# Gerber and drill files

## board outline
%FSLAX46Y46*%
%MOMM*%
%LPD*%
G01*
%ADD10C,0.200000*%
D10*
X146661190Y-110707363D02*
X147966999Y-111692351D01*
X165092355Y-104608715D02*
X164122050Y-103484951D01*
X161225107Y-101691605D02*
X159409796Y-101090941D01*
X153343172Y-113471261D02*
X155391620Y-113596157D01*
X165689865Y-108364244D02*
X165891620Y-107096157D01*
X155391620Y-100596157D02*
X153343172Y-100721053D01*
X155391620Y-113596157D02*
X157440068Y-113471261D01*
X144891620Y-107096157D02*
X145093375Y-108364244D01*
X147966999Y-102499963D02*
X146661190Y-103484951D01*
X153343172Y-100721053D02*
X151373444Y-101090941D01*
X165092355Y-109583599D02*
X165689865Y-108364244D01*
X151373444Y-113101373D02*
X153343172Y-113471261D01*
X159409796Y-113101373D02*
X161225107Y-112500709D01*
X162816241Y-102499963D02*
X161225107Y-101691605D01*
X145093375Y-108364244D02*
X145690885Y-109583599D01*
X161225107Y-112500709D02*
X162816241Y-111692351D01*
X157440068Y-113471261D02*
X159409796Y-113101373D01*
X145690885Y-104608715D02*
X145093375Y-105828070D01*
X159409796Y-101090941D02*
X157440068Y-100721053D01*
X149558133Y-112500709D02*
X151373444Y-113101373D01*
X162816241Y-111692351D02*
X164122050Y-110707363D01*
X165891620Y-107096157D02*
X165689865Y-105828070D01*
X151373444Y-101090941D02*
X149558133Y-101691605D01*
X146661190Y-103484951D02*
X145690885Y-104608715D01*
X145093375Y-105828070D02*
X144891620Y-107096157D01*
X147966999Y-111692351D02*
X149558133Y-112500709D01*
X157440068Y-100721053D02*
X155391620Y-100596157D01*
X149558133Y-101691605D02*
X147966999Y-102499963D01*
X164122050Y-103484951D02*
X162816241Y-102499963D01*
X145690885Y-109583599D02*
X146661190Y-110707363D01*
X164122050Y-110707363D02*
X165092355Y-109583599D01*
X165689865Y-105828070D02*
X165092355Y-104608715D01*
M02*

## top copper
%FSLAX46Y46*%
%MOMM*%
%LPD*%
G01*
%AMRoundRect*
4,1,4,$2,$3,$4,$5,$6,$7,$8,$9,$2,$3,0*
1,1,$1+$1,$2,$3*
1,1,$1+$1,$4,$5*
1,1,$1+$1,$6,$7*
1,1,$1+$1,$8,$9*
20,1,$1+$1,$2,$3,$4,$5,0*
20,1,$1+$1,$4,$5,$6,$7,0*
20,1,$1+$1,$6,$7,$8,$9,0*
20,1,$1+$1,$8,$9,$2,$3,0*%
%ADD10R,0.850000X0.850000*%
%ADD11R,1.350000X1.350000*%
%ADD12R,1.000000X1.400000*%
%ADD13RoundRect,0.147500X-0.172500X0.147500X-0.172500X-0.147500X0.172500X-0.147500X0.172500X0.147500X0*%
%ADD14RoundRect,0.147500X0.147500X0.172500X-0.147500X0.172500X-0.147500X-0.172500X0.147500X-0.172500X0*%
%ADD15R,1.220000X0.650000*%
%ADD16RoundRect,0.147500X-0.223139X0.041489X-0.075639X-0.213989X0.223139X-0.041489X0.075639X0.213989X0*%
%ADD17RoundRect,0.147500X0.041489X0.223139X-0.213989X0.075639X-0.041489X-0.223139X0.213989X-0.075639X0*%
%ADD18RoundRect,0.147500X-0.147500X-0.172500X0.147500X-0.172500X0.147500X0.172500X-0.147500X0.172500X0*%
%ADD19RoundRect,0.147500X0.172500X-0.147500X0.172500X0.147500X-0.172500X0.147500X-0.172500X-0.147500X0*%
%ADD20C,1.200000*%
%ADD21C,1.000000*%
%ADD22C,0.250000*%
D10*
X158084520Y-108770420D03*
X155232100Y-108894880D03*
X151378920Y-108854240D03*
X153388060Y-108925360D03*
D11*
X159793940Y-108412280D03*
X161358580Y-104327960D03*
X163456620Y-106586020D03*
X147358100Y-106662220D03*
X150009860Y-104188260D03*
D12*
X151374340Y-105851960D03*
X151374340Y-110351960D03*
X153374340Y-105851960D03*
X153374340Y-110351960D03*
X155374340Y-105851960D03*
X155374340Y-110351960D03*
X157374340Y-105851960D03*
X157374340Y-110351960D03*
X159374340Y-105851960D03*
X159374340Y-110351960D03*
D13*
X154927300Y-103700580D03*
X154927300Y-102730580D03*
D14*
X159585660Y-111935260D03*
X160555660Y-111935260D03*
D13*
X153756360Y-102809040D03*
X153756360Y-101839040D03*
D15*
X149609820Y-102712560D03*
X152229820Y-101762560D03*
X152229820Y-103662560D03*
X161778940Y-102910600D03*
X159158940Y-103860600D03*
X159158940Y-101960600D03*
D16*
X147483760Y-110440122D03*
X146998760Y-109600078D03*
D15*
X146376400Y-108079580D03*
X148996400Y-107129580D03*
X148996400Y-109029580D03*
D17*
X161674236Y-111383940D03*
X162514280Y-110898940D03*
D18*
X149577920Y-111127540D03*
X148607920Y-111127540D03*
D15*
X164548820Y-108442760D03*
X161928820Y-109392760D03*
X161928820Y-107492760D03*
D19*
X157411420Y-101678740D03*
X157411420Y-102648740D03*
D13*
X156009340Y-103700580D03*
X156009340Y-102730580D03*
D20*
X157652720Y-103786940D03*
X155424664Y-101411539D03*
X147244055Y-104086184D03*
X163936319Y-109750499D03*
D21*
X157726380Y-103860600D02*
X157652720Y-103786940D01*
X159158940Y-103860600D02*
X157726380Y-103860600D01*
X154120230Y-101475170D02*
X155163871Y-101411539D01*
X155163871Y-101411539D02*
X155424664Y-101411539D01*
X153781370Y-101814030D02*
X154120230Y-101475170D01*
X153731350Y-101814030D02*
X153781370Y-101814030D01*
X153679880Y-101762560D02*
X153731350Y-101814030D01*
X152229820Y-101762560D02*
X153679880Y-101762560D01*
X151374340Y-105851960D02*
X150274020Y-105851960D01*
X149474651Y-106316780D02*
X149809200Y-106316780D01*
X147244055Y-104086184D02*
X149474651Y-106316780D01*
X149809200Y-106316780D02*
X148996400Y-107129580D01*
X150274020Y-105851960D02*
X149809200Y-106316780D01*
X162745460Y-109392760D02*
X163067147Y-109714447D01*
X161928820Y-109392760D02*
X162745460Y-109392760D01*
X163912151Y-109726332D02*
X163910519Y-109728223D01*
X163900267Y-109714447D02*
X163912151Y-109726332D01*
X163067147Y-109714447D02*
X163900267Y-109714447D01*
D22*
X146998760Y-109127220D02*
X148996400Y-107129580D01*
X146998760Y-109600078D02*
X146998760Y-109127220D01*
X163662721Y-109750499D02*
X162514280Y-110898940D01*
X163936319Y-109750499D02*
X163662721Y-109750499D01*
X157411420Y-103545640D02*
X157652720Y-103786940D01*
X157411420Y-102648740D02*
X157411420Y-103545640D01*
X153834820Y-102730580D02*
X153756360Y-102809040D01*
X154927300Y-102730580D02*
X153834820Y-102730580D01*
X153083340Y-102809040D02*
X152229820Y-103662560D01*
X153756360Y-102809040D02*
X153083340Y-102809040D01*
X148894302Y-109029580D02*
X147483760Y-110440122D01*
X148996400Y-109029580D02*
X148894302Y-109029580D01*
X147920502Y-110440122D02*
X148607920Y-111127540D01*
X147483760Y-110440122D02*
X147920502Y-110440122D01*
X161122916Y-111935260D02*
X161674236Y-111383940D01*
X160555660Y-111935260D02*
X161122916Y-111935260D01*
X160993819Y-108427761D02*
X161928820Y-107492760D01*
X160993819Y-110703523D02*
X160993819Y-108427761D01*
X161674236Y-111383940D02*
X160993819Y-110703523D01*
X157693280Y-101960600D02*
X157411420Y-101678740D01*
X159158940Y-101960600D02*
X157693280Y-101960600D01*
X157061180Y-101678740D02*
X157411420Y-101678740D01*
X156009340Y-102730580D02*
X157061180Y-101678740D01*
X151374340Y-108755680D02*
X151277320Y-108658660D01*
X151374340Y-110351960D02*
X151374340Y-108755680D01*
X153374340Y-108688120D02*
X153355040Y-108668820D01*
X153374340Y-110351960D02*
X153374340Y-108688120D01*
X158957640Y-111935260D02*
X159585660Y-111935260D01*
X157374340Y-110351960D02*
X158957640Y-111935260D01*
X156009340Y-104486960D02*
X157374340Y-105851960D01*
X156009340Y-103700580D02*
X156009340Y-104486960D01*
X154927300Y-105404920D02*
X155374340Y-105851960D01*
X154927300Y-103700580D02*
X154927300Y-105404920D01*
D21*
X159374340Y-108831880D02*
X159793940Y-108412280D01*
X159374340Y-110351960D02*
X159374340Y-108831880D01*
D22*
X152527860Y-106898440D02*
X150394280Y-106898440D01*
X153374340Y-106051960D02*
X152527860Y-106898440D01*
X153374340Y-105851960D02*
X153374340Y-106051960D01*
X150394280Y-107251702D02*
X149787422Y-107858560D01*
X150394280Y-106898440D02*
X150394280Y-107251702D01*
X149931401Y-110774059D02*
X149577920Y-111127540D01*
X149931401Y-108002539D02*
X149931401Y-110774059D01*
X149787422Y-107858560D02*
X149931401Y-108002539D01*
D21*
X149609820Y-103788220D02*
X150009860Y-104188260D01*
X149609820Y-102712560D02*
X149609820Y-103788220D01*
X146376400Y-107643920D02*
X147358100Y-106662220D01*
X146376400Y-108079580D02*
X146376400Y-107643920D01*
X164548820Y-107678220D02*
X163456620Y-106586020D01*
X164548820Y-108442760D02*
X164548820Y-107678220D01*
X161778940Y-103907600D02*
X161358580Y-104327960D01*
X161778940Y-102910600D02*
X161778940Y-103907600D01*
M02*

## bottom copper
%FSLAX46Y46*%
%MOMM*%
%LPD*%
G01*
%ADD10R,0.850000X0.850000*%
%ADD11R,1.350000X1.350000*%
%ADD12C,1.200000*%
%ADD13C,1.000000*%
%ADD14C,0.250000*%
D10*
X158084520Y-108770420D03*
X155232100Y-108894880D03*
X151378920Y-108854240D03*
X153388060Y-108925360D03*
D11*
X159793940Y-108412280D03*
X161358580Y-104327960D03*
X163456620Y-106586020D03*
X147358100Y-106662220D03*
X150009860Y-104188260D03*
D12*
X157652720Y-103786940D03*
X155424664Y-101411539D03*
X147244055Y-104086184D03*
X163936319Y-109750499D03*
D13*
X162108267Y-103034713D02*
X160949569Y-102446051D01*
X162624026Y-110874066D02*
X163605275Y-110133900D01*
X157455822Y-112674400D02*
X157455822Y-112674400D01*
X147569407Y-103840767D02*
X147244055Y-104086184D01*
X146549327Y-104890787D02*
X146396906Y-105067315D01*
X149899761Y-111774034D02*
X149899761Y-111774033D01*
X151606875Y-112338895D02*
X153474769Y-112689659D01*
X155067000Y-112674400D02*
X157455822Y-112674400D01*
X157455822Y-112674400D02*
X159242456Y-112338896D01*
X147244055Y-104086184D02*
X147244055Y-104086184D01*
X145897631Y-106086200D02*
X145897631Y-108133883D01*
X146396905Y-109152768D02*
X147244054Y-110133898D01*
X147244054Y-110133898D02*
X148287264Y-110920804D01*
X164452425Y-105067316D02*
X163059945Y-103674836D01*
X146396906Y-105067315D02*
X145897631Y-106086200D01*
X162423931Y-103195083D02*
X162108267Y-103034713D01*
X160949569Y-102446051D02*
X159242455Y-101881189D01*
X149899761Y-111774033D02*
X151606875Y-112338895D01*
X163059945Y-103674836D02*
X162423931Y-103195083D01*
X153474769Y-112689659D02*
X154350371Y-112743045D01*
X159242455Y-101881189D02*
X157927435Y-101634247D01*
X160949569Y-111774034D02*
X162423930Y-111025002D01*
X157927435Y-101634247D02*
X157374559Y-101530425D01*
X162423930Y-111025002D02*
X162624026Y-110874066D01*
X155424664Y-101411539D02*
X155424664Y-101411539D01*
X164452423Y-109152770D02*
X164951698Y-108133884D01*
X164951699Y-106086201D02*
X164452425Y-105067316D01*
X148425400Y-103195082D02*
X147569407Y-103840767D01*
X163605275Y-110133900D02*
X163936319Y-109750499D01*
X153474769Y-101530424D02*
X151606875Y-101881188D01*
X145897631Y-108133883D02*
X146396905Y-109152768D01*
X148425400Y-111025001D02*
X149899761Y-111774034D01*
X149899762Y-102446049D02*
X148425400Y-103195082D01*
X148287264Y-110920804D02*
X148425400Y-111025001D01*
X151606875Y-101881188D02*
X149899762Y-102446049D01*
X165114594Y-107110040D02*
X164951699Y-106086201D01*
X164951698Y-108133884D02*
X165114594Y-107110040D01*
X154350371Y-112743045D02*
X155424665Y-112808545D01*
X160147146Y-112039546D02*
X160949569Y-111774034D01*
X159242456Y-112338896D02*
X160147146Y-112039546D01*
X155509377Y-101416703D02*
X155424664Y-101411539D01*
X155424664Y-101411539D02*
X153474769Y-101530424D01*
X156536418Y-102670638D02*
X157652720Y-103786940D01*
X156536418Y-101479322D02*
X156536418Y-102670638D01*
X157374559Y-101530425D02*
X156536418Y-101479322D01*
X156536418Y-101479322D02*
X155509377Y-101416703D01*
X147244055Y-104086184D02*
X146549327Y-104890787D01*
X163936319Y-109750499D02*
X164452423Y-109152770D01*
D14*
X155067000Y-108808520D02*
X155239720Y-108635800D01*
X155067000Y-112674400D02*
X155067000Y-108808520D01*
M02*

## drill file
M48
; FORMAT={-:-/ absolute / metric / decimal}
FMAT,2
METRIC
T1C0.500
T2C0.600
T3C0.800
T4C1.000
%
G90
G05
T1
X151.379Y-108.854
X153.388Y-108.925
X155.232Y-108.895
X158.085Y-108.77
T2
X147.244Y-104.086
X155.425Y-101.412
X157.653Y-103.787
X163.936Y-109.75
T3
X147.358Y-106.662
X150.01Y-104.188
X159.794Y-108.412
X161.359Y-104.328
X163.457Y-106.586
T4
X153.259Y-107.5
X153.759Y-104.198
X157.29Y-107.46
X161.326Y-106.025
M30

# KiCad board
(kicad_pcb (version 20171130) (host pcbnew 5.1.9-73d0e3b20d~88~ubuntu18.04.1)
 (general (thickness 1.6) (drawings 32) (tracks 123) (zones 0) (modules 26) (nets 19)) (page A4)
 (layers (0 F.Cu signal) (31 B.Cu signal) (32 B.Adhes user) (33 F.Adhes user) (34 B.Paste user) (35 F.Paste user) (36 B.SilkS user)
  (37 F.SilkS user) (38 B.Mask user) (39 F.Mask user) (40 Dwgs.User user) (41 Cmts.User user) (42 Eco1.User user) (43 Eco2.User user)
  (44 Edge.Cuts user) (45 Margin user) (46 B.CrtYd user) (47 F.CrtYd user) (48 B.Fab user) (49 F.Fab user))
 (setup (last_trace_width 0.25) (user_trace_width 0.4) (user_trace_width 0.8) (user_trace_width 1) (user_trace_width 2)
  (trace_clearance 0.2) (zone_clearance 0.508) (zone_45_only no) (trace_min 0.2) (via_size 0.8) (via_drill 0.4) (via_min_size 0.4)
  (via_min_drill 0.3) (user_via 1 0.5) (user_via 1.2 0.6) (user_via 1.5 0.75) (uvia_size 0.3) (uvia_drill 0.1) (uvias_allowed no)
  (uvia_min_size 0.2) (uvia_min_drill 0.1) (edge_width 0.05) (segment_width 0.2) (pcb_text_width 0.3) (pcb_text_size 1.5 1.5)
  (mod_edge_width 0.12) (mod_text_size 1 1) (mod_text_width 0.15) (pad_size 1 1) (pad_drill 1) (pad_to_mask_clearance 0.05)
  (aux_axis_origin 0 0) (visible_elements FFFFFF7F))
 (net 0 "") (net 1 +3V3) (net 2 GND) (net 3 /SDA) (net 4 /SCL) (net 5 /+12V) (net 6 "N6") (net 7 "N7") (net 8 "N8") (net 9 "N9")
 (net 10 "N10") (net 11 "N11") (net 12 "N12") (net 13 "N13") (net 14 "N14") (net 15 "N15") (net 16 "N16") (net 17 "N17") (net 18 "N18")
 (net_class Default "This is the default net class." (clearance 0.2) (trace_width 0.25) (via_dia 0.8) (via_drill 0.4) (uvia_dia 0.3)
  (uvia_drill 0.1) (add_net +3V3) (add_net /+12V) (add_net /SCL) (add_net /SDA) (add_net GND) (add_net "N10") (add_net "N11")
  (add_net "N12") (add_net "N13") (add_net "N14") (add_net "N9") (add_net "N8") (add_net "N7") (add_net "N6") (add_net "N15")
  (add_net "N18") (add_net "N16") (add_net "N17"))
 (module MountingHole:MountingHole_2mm (layer F.Cu) (at 157.2895 107.45978)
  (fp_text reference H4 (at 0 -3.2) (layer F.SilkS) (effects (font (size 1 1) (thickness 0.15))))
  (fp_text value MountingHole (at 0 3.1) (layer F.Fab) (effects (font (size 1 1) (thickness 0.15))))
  (pad "" np_thru_hole circle (at 0 0) (size 1 1) (drill 1) (layers *.Cu *.Mask)))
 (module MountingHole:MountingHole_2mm (layer F.Cu) (at 153.25852 107.50042)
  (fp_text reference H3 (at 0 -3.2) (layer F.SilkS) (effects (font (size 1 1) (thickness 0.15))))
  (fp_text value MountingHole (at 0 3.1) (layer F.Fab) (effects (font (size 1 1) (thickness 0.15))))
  (pad "" np_thru_hole circle (at 0 0) (size 1 1) (drill 1) (layers *.Cu *.Mask)))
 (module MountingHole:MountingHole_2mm (layer F.Cu) (at 153.7589 104.19842)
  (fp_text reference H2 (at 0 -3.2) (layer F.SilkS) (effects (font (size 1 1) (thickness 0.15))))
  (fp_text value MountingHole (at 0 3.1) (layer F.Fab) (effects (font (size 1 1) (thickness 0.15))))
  (pad "" np_thru_hole circle (at 0 0) (size 1 1) (drill 1) (layers *.Cu *.Mask)))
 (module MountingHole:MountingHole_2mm (layer F.Cu) (at 161.32556 106.02468)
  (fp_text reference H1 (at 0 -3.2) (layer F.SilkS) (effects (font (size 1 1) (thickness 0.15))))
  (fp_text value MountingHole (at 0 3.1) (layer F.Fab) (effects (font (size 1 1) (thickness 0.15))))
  (pad "" np_thru_hole circle (at 0 0) (size 1 1) (drill 1) (layers *.Cu *.Mask)))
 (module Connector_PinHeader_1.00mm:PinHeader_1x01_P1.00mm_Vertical (layer F.Cu) (at 158.08452 108.77042)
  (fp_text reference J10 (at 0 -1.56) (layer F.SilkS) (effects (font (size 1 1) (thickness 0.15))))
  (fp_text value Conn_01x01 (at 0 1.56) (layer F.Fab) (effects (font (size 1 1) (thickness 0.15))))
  (pad 1 thru_hole rect (at 0 0) (size 0.85 0.85) (drill 0.5) (layers *.Cu *.Mask) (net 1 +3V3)))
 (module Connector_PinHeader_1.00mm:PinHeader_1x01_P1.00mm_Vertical (layer F.Cu) (at 155.2321 108.89488)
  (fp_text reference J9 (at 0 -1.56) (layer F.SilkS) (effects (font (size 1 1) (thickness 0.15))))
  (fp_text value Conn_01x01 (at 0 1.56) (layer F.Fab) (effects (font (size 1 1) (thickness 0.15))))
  (pad 1 thru_hole rect (at 0 0) (size 0.85 0.85) (drill 0.5) (layers *.Cu *.Mask) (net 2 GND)))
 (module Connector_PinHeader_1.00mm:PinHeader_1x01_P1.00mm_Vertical (layer F.Cu) (at 151.37892 108.85424)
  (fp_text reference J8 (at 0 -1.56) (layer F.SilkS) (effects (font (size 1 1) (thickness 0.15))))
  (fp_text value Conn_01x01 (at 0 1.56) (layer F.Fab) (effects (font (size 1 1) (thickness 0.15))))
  (pad 1 thru_hole rect (at 0 0) (size 0.85 0.85) (drill 0.5) (layers *.Cu *.Mask) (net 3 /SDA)))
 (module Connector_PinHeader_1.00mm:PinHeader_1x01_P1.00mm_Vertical (layer F.Cu) (at 153.38806 108.92536)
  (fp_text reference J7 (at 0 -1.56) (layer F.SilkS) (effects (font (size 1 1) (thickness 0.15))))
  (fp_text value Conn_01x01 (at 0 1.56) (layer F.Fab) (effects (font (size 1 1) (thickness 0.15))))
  (pad 1 thru_hole rect (at 0 0) (size 0.85 0.85) (drill 0.5) (layers *.Cu *.Mask) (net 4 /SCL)))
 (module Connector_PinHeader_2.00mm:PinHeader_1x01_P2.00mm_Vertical (layer F.Cu) (at 159.79394 108.41228)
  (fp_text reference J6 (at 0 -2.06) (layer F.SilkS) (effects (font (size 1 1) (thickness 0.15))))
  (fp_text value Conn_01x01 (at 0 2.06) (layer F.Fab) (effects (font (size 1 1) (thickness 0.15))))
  (pad 1 thru_hole rect (at 0 0) (size 1.35 1.35) (drill 0.8) (layers *.Cu *.Mask) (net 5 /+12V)))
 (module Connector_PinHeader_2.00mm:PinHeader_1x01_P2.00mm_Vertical (layer F.Cu) (at 161.35858 104.32796)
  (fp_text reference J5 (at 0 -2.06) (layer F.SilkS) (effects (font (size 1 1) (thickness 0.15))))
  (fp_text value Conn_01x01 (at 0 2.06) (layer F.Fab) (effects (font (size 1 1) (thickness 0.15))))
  (pad 1 thru_hole rect (at 0 0) (size 1.35 1.35) (drill 0.8) (layers *.Cu *.Mask) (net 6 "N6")))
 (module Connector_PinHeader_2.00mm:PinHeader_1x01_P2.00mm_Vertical (layer F.Cu) (at 163.45662 106.58602)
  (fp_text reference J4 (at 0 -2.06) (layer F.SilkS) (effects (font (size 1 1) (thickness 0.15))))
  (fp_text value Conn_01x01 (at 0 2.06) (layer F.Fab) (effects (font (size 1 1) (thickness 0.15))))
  (pad 1 thru_hole rect (at 0 0) (size 1.35 1.35) (drill 0.8) (layers *.Cu *.Mask) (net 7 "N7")))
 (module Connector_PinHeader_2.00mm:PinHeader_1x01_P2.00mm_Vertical (layer F.Cu) (at 147.3581 106.66222)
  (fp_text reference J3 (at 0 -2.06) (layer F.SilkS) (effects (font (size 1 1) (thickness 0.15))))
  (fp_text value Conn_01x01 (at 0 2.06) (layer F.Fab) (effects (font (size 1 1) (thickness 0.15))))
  (pad 1 thru_hole rect (at 0 0) (size 1.35 1.35) (drill 0.8) (layers *.Cu *.Mask) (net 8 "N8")))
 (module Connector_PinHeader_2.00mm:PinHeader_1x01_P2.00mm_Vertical (layer F.Cu) (at 150.00986 104.18826)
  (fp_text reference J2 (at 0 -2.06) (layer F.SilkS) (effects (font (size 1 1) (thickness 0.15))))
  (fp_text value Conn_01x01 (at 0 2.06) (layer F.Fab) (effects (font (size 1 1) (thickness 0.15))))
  (pad 1 thru_hole rect (at 0 0) (size 1.35 1.35) (drill 0.8) (layers *.Cu *.Mask) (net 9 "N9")))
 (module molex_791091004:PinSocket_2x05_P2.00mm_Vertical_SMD (layer F.Cu) (at 155.37434 108.10196 90)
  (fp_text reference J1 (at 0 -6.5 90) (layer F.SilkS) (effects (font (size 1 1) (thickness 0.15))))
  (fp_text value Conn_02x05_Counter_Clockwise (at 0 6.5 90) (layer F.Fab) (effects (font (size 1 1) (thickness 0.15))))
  (pad 1 smd rect (at 2.25 -4 90) (size 1.4 1) (layers F.Cu F.Paste F.Mask) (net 2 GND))
  (pad 2 smd rect (at -2.25 -4 90) (size 1.4 1) (layers F.Cu F.Paste F.Mask) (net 3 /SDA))
  (pad 3 smd rect (at 2.25 -2 90) (size 1.4 1) (layers F.Cu F.Paste F.Mask) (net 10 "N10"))
  (pad 4 smd rect (at -2.25 -2 90) (size 1.4 1) (layers F.Cu F.Paste F.Mask) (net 4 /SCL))
  (pad 5 smd rect (at 2.25 0 90) (size 1.4 1) (layers F.Cu F.Paste F.Mask) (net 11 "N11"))
  (pad 6 smd rect (at -2.25 0 90) (size 1.4 1) (layers F.Cu F.Paste F.Mask) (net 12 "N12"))
  (pad 7 smd rect (at 2.25 2 90) (size 1.4 1) (layers F.Cu F.Paste F.Mask) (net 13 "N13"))
  (pad 8 smd rect (at -2.25 2 90) (size 1.4 1) (layers F.Cu F.Paste F.Mask) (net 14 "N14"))
  (pad 9 smd rect (at 2.25 4 90) (size 1.4 1) (layers F.Cu F.Paste F.Mask) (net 1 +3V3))
  (pad 10 smd rect (at -2.25 4 90) (size 1.4 1) (layers F.Cu F.Paste F.Mask) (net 5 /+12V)))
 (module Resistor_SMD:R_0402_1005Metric (layer F.Cu) (at 154.9273 103.21558 270)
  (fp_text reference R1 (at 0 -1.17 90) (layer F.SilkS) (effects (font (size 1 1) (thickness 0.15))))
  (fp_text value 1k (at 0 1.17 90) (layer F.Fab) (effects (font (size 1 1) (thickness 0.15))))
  (pad 2 smd roundrect (at 0.485 0 270) (size 0.59 0.64) (layers F.Cu F.Paste F.Mask) (roundrect_rratio 0.25) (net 11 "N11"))
  (pad 1 smd roundrect (at -0.485 0 270) (size 0.59 0.64) (layers F.Cu F.Paste F.Mask) (roundrect_rratio 0.25) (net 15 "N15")))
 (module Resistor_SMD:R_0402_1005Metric (layer F.Cu) (at 160.07066 111.93526 180)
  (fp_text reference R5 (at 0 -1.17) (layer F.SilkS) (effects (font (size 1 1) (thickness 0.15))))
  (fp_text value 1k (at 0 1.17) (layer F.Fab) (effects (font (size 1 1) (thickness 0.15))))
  (pad 2 smd roundrect (at 0.485 0 180) (size 0.59 0.64) (layers F.Cu F.Paste F.Mask) (roundrect_rratio 0.25) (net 14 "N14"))
  (pad 1 smd roundrect (at -0.485 0 180) (size 0.59 0.64) (layers F.Cu F.Paste F.Mask) (roundrect_rratio 0.25) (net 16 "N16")))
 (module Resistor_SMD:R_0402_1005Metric (layer F.Cu) (at 153.75636 102.32404 270)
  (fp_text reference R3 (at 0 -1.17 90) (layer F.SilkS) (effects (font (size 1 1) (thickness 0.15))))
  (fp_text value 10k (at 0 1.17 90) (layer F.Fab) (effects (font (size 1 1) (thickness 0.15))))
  (pad 2 smd roundrect (at 0.485 0 270) (size 0.59 0.64) (layers F.Cu F.Paste F.Mask) (roundrect_rratio 0.25) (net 15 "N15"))
  (pad 1 smd roundrect (at -0.485 0 270) (size 0.59 0.64) (layers F.Cu F.Paste F.Mask) (roundrect_rratio 0.25) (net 2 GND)))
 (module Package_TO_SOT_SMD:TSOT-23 (layer F.Cu) (at 150.91982 102.71256 180)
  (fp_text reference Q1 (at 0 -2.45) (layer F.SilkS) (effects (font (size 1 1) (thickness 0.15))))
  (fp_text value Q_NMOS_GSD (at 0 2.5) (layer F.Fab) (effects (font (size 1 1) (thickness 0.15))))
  (pad 3 smd rect (at 1.31 0 180) (size 1.22 0.65) (layers F.Cu F.Paste F.Mask) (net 9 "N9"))
  (pad 2 smd rect (at -1.31 0.95 180) (size 1.22 0.65) (layers F.Cu F.Paste F.Mask) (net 2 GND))
  (pad 1 smd rect (at -1.31 -0.95 180) (size 1.22 0.65) (layers F.Cu F.Paste F.Mask) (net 15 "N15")))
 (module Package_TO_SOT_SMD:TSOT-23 (layer F.Cu) (at 160.46894 102.9106)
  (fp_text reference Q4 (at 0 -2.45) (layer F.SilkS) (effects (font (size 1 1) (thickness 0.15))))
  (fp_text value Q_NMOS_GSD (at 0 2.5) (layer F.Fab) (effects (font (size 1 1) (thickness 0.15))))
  (pad 3 smd rect (at 1.31 0) (size 1.22 0.65) (layers F.Cu F.Paste F.Mask) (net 6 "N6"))
  (pad 2 smd rect (at -1.31 0.95) (size 1.22 0.65) (layers F.Cu F.Paste F.Mask) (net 2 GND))
  (pad 1 smd rect (at -1.31 -0.95) (size 1.22 0.65) (layers F.Cu F.Paste F.Mask) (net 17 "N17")))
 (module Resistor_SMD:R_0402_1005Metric (layer F.Cu) (at 147.24126 110.0201 300)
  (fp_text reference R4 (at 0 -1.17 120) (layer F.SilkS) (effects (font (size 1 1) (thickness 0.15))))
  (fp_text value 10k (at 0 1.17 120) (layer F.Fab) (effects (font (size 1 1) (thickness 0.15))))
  (pad 2 smd roundrect (at 0.485 0 300) (size 0.59 0.64) (layers F.Cu F.Paste F.Mask) (roundrect_rratio 0.25) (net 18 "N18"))
  (pad 1 smd roundrect (at -0.485 0 300) (size 0.59 0.64) (layers F.Cu F.Paste F.Mask) (roundrect_rratio 0.25) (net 2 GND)))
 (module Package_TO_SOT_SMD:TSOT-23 (layer F.Cu) (at 147.6864 108.07958 180)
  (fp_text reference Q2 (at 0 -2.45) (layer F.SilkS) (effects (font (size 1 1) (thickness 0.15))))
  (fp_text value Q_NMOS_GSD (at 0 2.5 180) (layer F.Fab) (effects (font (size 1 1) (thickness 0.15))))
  (pad 3 smd rect (at 1.31 0 180) (size 1.22 0.65) (layers F.Cu F.Paste F.Mask) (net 8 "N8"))
  (pad 2 smd rect (at -1.31 0.95 180) (size 1.22 0.65) (layers F.Cu F.Paste F.Mask) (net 2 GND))
  (pad 1 smd rect (at -1.31 -0.95 180) (size 1.22 0.65) (layers F.Cu F.Paste F.Mask) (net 18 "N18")))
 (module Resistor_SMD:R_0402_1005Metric (layer F.Cu) (at 162.094258 111.14144 210)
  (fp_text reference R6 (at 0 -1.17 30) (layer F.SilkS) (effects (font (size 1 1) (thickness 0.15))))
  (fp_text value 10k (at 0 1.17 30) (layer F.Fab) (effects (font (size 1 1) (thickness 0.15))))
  (pad 2 smd roundrect (at 0.485 0 210) (size 0.59 0.64) (layers F.Cu F.Paste F.Mask) (roundrect_rratio 0.25) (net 16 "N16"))
  (pad 1 smd roundrect (at -0.485 0 210) (size 0.59 0.64) (layers F.Cu F.Paste F.Mask) (roundrect_rratio 0.25) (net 2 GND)))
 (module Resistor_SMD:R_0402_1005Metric (layer F.Cu) (at 149.09292 111.12754)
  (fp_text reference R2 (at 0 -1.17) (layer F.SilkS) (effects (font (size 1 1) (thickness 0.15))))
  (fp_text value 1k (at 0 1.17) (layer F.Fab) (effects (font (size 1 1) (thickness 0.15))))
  (pad 2 smd roundrect (at 0.485 0) (size 0.59 0.64) (layers F.Cu F.Paste F.Mask) (roundrect_rratio 0.25) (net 10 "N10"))
  (pad 1 smd roundrect (at -0.485 0) (size 0.59 0.64) (layers F.Cu F.Paste F.Mask) (roundrect_rratio 0.25) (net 18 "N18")))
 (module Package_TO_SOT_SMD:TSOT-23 (layer F.Cu) (at 163.23882 108.44276)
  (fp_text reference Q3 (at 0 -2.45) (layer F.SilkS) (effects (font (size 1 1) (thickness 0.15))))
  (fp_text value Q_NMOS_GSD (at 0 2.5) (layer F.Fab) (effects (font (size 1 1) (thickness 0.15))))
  (pad 3 smd rect (at 1.31 0) (size 1.22 0.65) (layers F.Cu F.Paste F.Mask) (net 7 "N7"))
  (pad 2 smd rect (at -1.31 0.95) (size 1.22 0.65) (layers F.Cu F.Paste F.Mask) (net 2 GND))
  (pad 1 smd rect (at -1.31 -0.95) (size 1.22 0.65) (layers F.Cu F.Paste F.Mask) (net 16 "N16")))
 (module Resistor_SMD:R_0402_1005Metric (layer F.Cu) (at 157.41142 102.16374 90)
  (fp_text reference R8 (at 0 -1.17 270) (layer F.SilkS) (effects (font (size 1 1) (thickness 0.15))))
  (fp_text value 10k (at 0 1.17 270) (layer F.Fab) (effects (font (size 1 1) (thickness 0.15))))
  (pad 2 smd roundrect (at 0.485 0 90) (size 0.59 0.64) (layers F.Cu F.Paste F.Mask) (roundrect_rratio 0.25) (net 17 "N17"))
  (pad 1 smd roundrect (at -0.485 0 90) (size 0.59 0.64) (layers F.Cu F.Paste F.Mask) (roundrect_rratio 0.25) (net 2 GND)))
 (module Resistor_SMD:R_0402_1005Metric (layer F.Cu) (at 156.00934 103.21558 270)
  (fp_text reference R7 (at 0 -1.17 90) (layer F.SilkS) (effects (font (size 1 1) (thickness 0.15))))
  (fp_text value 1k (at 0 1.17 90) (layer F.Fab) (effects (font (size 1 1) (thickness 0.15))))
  (pad 2 smd roundrect (at 0.485 0 270) (size 0.59 0.64) (layers F.Cu F.Paste F.Mask) (roundrect_rratio 0.25) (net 13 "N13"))
  (pad 1 smd roundrect (at -0.485 0 270) (size 0.59 0.64) (layers F.Cu F.Paste F.Mask) (roundrect_rratio 0.25) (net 17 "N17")))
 (gr_line (start 146.66119 110.707363) (end 147.966999 111.692351) (layer Edge.Cuts) (width 0.2))
 (gr_line (start 165.092355 104.608715) (end 164.12205 103.484951) (layer Edge.Cuts) (width 0.2))
 (gr_line (start 161.225107 101.691605) (end 159.409796 101.090941) (layer Edge.Cuts) (width 0.2))
 (gr_line (start 153.343172 113.471261) (end 155.39162 113.596157) (layer Edge.Cuts) (width 0.2))
 (gr_line (start 165.689865 108.364244) (end 165.89162 107.096157) (layer Edge.Cuts) (width 0.2))
 (gr_line (start 155.39162 100.596157) (end 153.343172 100.721053) (layer Edge.Cuts) (width 0.2))
 (gr_line (start 155.39162 113.596157) (end 157.440068 113.471261) (layer Edge.Cuts) (width 0.2))
 (gr_line (start 144.89162 107.096157) (end 145.093375 108.364244) (layer Edge.Cuts) (width 0.2))
 (gr_line (start 147.966999 102.499963) (end 146.66119 103.484951) (layer Edge.Cuts) (width 0.2))
 (gr_line (start 153.343172 100.721053) (end 151.373444 101.090941) (layer Edge.Cuts) (width 0.2))
 (gr_line (start 165.092355 109.583599) (end 165.689865 108.364244) (layer Edge.Cuts) (width 0.2))
 (gr_line (start 151.373444 113.101373) (end 153.343172 113.471261) (layer Edge.Cuts) (width 0.2))
 (gr_line (start 159.409796 113.101373) (end 161.225107 112.500709) (layer Edge.Cuts) (width 0.2))
 (gr_line (start 162.816241 102.499963) (end 161.225107 101.691605) (layer Edge.Cuts) (width 0.2))
 (gr_line (start 145.093375 108.364244) (end 145.690885 109.583599) (layer Edge.Cuts) (width 0.2))
 (gr_line (start 161.225107 112.500709) (end 162.816241 111.692351) (layer Edge.Cuts) (width 0.2))
 (gr_line (start 157.440068 113.471261) (end 159.409796 113.101373) (layer Edge.Cuts) (width 0.2))
 (gr_line (start 145.690885 104.608715) (end 145.093375 105.82807) (layer Edge.Cuts) (width 0.2))
 (gr_line (start 159.409796 101.090941) (end 157.440068 100.721053) (layer Edge.Cuts) (width 0.2))
 (gr_line (start 149.558133 112.500709) (end 151.373444 113.101373) (layer Edge.Cuts) (width 0.2))
 (gr_line (start 162.816241 111.692351) (end 164.12205 110.707363) (layer Edge.Cuts) (width 0.2))
 (gr_line (start 165.89162 107.096157) (end 165.689865 105.82807) (layer Edge.Cuts) (width 0.2))
 (gr_line (start 151.373444 101.090941) (end 149.558133 101.691605) (layer Edge.Cuts) (width 0.2))
 (gr_line (start 146.66119 103.484951) (end 145.690885 104.608715) (layer Edge.Cuts) (width 0.2))
 (gr_line (start 145.093375 105.82807) (end 144.89162 107.096157) (layer Edge.Cuts) (width 0.2))
 (gr_line (start 147.966999 111.692351) (end 149.558133 112.500709) (layer Edge.Cuts) (width 0.2))
 (gr_line (start 157.440068 100.721053) (end 155.39162 100.596157) (layer Edge.Cuts) (width 0.2))
 (gr_line (start 149.558133 101.691605) (end 147.966999 102.499963) (layer Edge.Cuts) (width 0.2))
 (gr_line (start 164.12205 103.484951) (end 162.816241 102.499963) (layer Edge.Cuts) (width 0.2))
 (gr_line (start 145.690885 109.583599) (end 146.66119 110.707363) (layer Edge.Cuts) (width 0.2))
 (gr_line (start 164.12205 110.707363) (end 165.092355 109.583599) (layer Edge.Cuts) (width 0.2))
 (gr_line (start 165.689865 105.82807) (end 165.092355 104.608715) (layer Edge.Cuts) (width 0.2))
 (segment (start 162.108267 103.034713) (end 160.949569 102.446051) (width 1) (layer B.Cu) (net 2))
 (segment (start 162.624026 110.874066) (end 163.605275 110.1339) (width 1) (layer B.Cu) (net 2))
 (segment (start 157.455822 112.6744) (end 157.455822 112.6744) (width 1) (layer B.Cu) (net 2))
 (segment (start 147.569407 103.840767) (end 147.244055 104.086184) (width 1) (layer B.Cu) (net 2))
 (segment (start 146.549327 104.890787) (end 146.396906 105.067315) (width 1) (layer B.Cu) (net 2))
 (segment (start 149.899761 111.774034) (end 149.899761 111.774033) (width 1) (layer B.Cu) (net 2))
 (segment (start 151.606875 112.338895) (end 153.474769 112.689659) (width 1) (layer B.Cu) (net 2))
 (segment (start 155.067 112.6744) (end 157.455822 112.6744) (width 1) (layer B.Cu) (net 2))
 (segment (start 157.455822 112.6744) (end 159.242456 112.338896) (width 1) (layer B.Cu) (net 2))
 (segment (start 147.244055 104.086184) (end 147.244055 104.086184) (width 1) (layer B.Cu) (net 2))
 (segment (start 145.897631 106.0862) (end 145.897631 108.133883) (width 1) (layer B.Cu) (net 2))
 (segment (start 146.396905 109.152768) (end 147.244054 110.133898) (width 1) (layer B.Cu) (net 2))
 (segment (start 147.244054 110.133898) (end 148.287264 110.920804) (width 1) (layer B.Cu) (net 2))
 (segment (start 164.452425 105.067316) (end 163.059945 103.674836) (width 1) (layer B.Cu) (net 2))
 (segment (start 146.396906 105.067315) (end 145.897631 106.0862) (width 1) (layer B.Cu) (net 2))
 (segment (start 162.423931 103.195083) (end 162.108267 103.034713) (width 1) (layer B.Cu) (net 2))
 (segment (start 160.949569 102.446051) (end 159.242455 101.881189) (width 1) (layer B.Cu) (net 2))
 (segment (start 149.899761 111.774033) (end 151.606875 112.338895) (width 1) (layer B.Cu) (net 2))
 (segment (start 163.059945 103.674836) (end 162.423931 103.195083) (width 1) (layer B.Cu) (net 2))
 (segment (start 153.474769 112.689659) (end 154.350371 112.743045) (width 1) (layer B.Cu) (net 2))
 (segment (start 159.242455 101.881189) (end 157.927435 101.634247) (width 1) (layer B.Cu) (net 2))
 (segment (start 160.949569 111.774034) (end 162.42393 111.025002) (width 1) (layer B.Cu) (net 2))
 (segment (start 157.927435 101.634247) (end 157.374559 101.530425) (width 1) (layer B.Cu) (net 2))
 (segment (start 162.42393 111.025002) (end 162.624026 110.874066) (width 1) (layer B.Cu) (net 2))
 (segment (start 155.424664 101.411539) (end 155.424664 101.411539) (width 1) (layer B.Cu) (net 2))
 (segment (start 164.452423 109.15277) (end 164.951698 108.133884) (width 1) (layer B.Cu) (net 2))
 (segment (start 164.951699 106.086201) (end 164.452425 105.067316) (width 1) (layer B.Cu) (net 2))
 (segment (start 148.4254 103.195082) (end 147.569407 103.840767) (width 1) (layer B.Cu) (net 2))
 (segment (start 163.605275 110.1339) (end 163.936319 109.750499) (width 1) (layer B.Cu) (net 2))
 (segment (start 153.474769 101.530424) (end 151.606875 101.881188) (width 1) (layer B.Cu) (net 2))
 (segment (start 145.897631 108.133883) (end 146.396905 109.152768) (width 1) (layer B.Cu) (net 2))
 (segment (start 148.4254 111.025001) (end 149.899761 111.774034) (width 1) (layer B.Cu) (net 2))
 (segment (start 149.899762 102.446049) (end 148.4254 103.195082) (width 1) (layer B.Cu) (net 2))
 (segment (start 148.287264 110.920804) (end 148.4254 111.025001) (width 1) (layer B.Cu) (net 2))
 (segment (start 151.606875 101.881188) (end 149.899762 102.446049) (width 1) (layer B.Cu) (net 2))
 (segment (start 165.114594 107.11004) (end 164.951699 106.086201) (width 1) (layer B.Cu) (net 2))
 (segment (start 164.951698 108.133884) (end 165.114594 107.11004) (width 1) (layer B.Cu) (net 2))
 (segment (start 154.350371 112.743045) (end 155.424665 112.808545) (width 1) (layer B.Cu) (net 2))
 (segment (start 160.147146 112.039546) (end 160.949569 111.774034) (width 1) (layer B.Cu) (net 2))
 (segment (start 159.242456 112.338896) (end 160.147146 112.039546) (width 1) (layer B.Cu) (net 2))
 (segment (start 155.509377 101.416703) (end 155.424664 101.411539) (width 1) (layer B.Cu) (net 2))
 (via (at 157.65272 103.78694) (size 1.2) (drill 0.6) (layers F.Cu B.Cu) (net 2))
 (segment (start 155.424664 101.411539) (end 153.474769 101.530424) (width 1) (layer B.Cu) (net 2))
 (via (at 155.424664 101.411539) (size 1.2) (drill 0.6) (layers F.Cu B.Cu) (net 2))
 (segment (start 156.536418 102.670638) (end 157.65272 103.78694) (width 1) (layer B.Cu) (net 2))
 (segment (start 156.536418 101.479322) (end 156.536418 102.670638) (width 1) (layer B.Cu) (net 2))
 (segment (start 157.374559 101.530425) (end 156.536418 101.479322) (width 1) (layer B.Cu) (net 2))
 (segment (start 156.536418 101.479322) (end 155.509377 101.416703) (width 1) (layer B.Cu) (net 2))
 (segment (start 157.72638 103.8606) (end 157.65272 103.78694) (width 1) (layer F.Cu) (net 2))
 (segment (start 159.15894 103.8606) (end 157.72638 103.8606) (width 1) (layer F.Cu) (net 2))
 (segment (start 154.12023 101.47517) (end 155.163871 101.411539) (width 1) (layer F.Cu) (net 2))
 (segment (start 155.163871 101.411539) (end 155.424664 101.411539) (width 1) (layer F.Cu) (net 2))
 (segment (start 153.78137 101.81403) (end 154.12023 101.47517) (width 1) (layer F.Cu) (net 2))
 (segment (start 153.73135 101.81403) (end 153.78137 101.81403) (width 1) (layer F.Cu) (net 2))
 (segment (start 153.67988 101.76256) (end 153.73135 101.81403) (width 1) (layer F.Cu) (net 2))
 (segment (start 152.22982 101.76256) (end 153.67988 101.76256) (width 1) (layer F.Cu) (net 2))
 (segment (start 151.37434 105.85196) (end 150.27402 105.85196) (width 1) (layer F.Cu) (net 2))
 (segment (start 147.244055 104.086184) (end 146.549327 104.890787) (width 1) (layer B.Cu) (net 2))
 (via (at 147.244055 104.086184) (size 1.2) (drill 0.6) (layers F.Cu B.Cu) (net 2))
 (segment (start 149.474651 106.31678) (end 149.8092 106.31678) (width 1) (layer F.Cu) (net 2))
 (segment (start 147.244055 104.086184) (end 149.474651 106.31678) (width 1) (layer F.Cu) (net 2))
 (segment (start 149.8092 106.31678) (end 148.9964 107.12958) (width 1) (layer F.Cu) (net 2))
 (segment (start 150.27402 105.85196) (end 149.8092 106.31678) (width 1) (layer F.Cu) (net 2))
 (segment (start 163.936319 109.750499) (end 164.452423 109.15277) (width 1) (layer B.Cu) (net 2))
 (via (at 163.936319 109.750499) (size 1.2) (drill 0.6) (layers F.Cu B.Cu) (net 2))
 (segment (start 162.74546 109.39276) (end 163.067147 109.714447) (width 1) (layer F.Cu) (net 2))
 (segment (start 161.92882 109.39276) (end 162.74546 109.39276) (width 1) (layer F.Cu) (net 2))
 (segment (start 163.912151 109.726332) (end 163.910519 109.728223) (width 1) (layer F.Cu) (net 2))
 (segment (start 163.900267 109.714447) (end 163.912151 109.726332) (width 1) (layer F.Cu) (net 2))
 (segment (start 163.067147 109.714447) (end 163.900267 109.714447) (width 1) (layer F.Cu) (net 2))
 (segment (start 146.99876 109.12722) (end 148.9964 107.12958) (width 0.25) (layer F.Cu) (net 2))
 (segment (start 146.99876 109.600078) (end 146.99876 109.12722) (width 0.25) (layer F.Cu) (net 2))
 (segment (start 163.662721 109.750499) (end 162.51428 110.89894) (width 0.25) (layer F.Cu) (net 2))
 (segment (start 163.936319 109.750499) (end 163.662721 109.750499) (width 0.25) (layer F.Cu) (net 2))
 (segment (start 157.41142 103.54564) (end 157.65272 103.78694) (width 0.25) (layer F.Cu) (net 2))
 (segment (start 157.41142 102.64874) (end 157.41142 103.54564) (width 0.25) (layer F.Cu) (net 2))
 (segment (start 155.067 108.80852) (end 155.23972 108.6358) (width 0.25) (layer B.Cu) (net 2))
 (segment (start 155.067 112.6744) (end 155.067 108.80852) (width 0.25) (layer B.Cu) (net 2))
 (segment (start 153.83482 102.73058) (end 153.75636 102.80904) (width 0.25) (layer F.Cu) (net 15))
 (segment (start 154.9273 102.73058) (end 153.83482 102.73058) (width 0.25) (layer F.Cu) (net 15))
 (segment (start 153.08334 102.80904) (end 152.22982 103.66256) (width 0.25) (layer F.Cu) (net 15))
 (segment (start 153.75636 102.80904) (end 153.08334 102.80904) (width 0.25) (layer F.Cu) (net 15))
 (segment (start 148.894302 109.02958) (end 147.48376 110.440122) (width 0.25) (layer F.Cu) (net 18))
 (segment (start 148.9964 109.02958) (end 148.894302 109.02958) (width 0.25) (layer F.Cu) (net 18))
 (segment (start 147.920502 110.440122) (end 148.60792 111.12754) (width 0.25) (layer F.Cu) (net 18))
 (segment (start 147.48376 110.440122) (end 147.920502 110.440122) (width 0.25) (layer F.Cu) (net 18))
 (segment (start 161.122916 111.93526) (end 161.674236 111.38394) (width 0.25) (layer F.Cu) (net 16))
 (segment (start 160.55566 111.93526) (end 161.122916 111.93526) (width 0.25) (layer F.Cu) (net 16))
 (segment (start 160.993819 108.427761) (end 161.92882 107.49276) (width 0.25) (layer F.Cu) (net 16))
 (segment (start 160.993819 110.703523) (end 160.993819 108.427761) (width 0.25) (layer F.Cu) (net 16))
 (segment (start 161.674236 111.38394) (end 160.993819 110.703523) (width 0.25) (layer F.Cu) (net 16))
 (segment (start 157.69328 101.9606) (end 157.41142 101.67874) (width 0.25) (layer F.Cu) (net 17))
 (segment (start 159.15894 101.9606) (end 157.69328 101.9606) (width 0.25) (layer F.Cu) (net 17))
 (segment (start 157.06118 101.67874) (end 157.41142 101.67874) (width 0.25) (layer F.Cu) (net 17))
 (segment (start 156.00934 102.73058) (end 157.06118 101.67874) (width 0.25) (layer F.Cu) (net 17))
 (segment (start 151.37434 108.75568) (end 151.27732 108.65866) (width 0.25) (layer F.Cu) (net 3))
 (segment (start 151.37434 110.35196) (end 151.37434 108.75568) (width 0.25) (layer F.Cu) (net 3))
 (segment (start 153.37434 108.68812) (end 153.35504 108.66882) (width 0.25) (layer F.Cu) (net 4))
 (segment (start 153.37434 110.35196) (end 153.37434 108.68812) (width 0.25) (layer F.Cu) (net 4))
 (segment (start 158.95764 111.93526) (end 159.58566 111.93526) (width 0.25) (layer F.Cu) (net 14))
 (segment (start 157.37434 110.35196) (end 158.95764 111.93526) (width 0.25) (layer F.Cu) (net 14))
 (segment (start 156.00934 104.48696) (end 157.37434 105.85196) (width 0.25) (layer F.Cu) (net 13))
 (segment (start 156.00934 103.70058) (end 156.00934 104.48696) (width 0.25) (layer F.Cu) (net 13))
 (segment (start 154.9273 105.40492) (end 155.37434 105.85196) (width 0.25) (layer F.Cu) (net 11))
 (segment (start 154.9273 103.70058) (end 154.9273 105.40492) (width 0.25) (layer F.Cu) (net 11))
 (segment (start 159.37434 108.83188) (end 159.79394 108.41228) (width 1) (layer F.Cu) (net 5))
 (segment (start 159.37434 110.35196) (end 159.37434 108.83188) (width 1) (layer F.Cu) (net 5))
 (segment (start 152.52786 106.89844) (end 150.39428 106.89844) (width 0.25) (layer F.Cu) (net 10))
 (segment (start 153.37434 106.05196) (end 152.52786 106.89844) (width 0.25) (layer F.Cu) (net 10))
 (segment (start 153.37434 105.85196) (end 153.37434 106.05196) (width 0.25) (layer F.Cu) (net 10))
 (segment (start 150.39428 107.251702) (end 149.787422 107.85856) (width 0.25) (layer F.Cu) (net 10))
 (segment (start 150.39428 106.89844) (end 150.39428 107.251702) (width 0.25) (layer F.Cu) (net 10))
 (segment (start 149.931401 110.774059) (end 149.57792 111.12754) (width 0.25) (layer F.Cu) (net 10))
 (segment (start 149.931401 108.002539) (end 149.931401 110.774059) (width 0.25) (layer F.Cu) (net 10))
 (segment (start 149.787422 107.85856) (end 149.931401 108.002539) (width 0.25) (layer F.Cu) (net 10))
 (segment (start 149.60982 103.78822) (end 150.00986 104.18826) (width 1) (layer F.Cu) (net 9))
 (segment (start 149.60982 102.71256) (end 149.60982 103.78822) (width 1) (layer F.Cu) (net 9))
 (segment (start 146.3764 107.64392) (end 147.3581 106.66222) (width 1) (layer F.Cu) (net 8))
 (segment (start 146.3764 108.07958) (end 146.3764 107.64392) (width 1) (layer F.Cu) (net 8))
 (segment (start 164.54882 107.67822) (end 163.45662 106.58602) (width 1) (layer F.Cu) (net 7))
 (segment (start 164.54882 108.44276) (end 164.54882 107.67822) (width 1) (layer F.Cu) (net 7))
 (segment (start 161.77894 103.9076) (end 161.35858 104.32796) (width 1) (layer F.Cu) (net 6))
 (segment (start 161.77894 102.9106) (end 161.77894 103.9076) (width 1) (layer F.Cu) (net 6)))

